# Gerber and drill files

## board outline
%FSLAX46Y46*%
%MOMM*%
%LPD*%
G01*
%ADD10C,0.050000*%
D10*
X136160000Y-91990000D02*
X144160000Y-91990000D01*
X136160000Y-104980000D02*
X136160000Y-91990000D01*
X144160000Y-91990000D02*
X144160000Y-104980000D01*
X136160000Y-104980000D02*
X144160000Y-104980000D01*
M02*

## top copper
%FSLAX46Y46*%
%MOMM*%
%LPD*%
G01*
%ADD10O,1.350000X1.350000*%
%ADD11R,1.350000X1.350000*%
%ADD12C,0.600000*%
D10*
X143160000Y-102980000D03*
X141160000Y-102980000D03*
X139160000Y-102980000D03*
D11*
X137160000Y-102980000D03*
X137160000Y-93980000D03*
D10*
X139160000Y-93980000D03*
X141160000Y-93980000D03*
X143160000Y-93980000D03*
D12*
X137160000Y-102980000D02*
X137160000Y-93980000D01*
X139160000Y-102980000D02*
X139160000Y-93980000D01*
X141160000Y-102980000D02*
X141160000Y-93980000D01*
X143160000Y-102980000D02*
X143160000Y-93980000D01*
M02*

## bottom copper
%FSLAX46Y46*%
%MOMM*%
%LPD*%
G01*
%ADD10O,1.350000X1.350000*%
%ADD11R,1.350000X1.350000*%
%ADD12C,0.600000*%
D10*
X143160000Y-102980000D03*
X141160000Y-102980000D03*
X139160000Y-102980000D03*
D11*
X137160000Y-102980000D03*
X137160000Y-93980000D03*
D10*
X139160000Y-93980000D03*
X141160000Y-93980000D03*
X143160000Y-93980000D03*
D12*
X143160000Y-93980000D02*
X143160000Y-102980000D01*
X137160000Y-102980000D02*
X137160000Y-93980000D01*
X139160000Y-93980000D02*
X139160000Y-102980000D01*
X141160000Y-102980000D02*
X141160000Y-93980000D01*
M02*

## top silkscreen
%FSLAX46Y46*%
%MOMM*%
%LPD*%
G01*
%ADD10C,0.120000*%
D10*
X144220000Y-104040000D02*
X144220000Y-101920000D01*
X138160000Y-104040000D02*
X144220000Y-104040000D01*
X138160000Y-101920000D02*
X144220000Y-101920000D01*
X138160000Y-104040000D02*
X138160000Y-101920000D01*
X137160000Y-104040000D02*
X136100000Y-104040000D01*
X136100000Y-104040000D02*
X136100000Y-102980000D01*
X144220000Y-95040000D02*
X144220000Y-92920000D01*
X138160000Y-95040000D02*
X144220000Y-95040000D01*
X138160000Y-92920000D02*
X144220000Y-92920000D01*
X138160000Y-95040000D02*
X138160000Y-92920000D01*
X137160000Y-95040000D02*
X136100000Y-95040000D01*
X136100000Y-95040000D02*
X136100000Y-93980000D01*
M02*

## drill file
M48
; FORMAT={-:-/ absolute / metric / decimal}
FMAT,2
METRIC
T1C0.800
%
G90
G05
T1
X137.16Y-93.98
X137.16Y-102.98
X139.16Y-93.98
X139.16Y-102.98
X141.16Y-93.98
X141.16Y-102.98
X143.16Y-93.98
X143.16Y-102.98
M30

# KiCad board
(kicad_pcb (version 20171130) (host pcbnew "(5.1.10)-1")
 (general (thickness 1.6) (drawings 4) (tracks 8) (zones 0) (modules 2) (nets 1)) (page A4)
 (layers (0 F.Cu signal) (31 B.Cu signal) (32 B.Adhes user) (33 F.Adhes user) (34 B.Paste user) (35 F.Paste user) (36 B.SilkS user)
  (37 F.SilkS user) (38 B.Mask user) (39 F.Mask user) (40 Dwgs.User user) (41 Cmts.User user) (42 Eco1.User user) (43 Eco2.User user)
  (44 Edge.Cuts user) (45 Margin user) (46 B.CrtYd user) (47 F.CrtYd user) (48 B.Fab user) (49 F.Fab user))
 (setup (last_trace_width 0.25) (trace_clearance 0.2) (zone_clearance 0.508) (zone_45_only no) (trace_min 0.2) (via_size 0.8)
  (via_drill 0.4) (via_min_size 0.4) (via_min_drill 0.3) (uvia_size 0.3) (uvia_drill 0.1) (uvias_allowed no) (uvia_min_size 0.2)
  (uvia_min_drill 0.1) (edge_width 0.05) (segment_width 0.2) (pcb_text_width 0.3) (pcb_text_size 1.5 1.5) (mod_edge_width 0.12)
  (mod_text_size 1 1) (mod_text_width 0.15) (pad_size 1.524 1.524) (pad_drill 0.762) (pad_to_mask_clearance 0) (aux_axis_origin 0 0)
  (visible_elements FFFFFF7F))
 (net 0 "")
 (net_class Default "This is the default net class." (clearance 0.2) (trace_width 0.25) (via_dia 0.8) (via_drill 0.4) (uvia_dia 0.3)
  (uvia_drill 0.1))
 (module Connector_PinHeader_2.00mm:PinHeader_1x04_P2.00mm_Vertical (layer F.Cu) (at 137.16 102.98 90)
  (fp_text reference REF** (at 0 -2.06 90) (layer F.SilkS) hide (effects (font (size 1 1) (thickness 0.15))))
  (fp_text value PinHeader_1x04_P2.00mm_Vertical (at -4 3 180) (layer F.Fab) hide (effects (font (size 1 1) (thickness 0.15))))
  (fp_line (start -1.06 7.06) (end 1.06 7.06) (layer F.SilkS) (width 0.12))
  (fp_line (start -1.06 1) (end -1.06 7.06) (layer F.SilkS) (width 0.12))
  (fp_line (start 1.06 1) (end 1.06 7.06) (layer F.SilkS) (width 0.12))
  (fp_line (start -1.06 1) (end 1.06 1) (layer F.SilkS) (width 0.12))
  (fp_line (start -1.06 0) (end -1.06 -1.06) (layer F.SilkS) (width 0.12))
  (fp_line (start -1.06 -1.06) (end 0 -1.06) (layer F.SilkS) (width 0.12))
  (pad 4 thru_hole oval (at 0 6 90) (size 1.35 1.35) (drill 0.8) (layers *.Cu *.Mask))
  (pad 3 thru_hole oval (at 0 4 90) (size 1.35 1.35) (drill 0.8) (layers *.Cu *.Mask))
  (pad 2 thru_hole oval (at 0 2 90) (size 1.35 1.35) (drill 0.8) (layers *.Cu *.Mask))
  (pad 1 thru_hole rect (at 0 0 90) (size 1.35 1.35) (drill 0.8) (layers *.Cu *.Mask)))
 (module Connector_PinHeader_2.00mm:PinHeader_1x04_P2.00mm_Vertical (layer F.Cu) (at 137.16 93.98 90)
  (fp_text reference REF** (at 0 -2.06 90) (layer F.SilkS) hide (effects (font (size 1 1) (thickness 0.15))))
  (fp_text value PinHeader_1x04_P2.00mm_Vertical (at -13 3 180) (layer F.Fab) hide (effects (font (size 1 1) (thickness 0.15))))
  (fp_line (start -1.06 7.06) (end 1.06 7.06) (layer F.SilkS) (width 0.12))
  (fp_line (start -1.06 1) (end -1.06 7.06) (layer F.SilkS) (width 0.12))
  (fp_line (start 1.06 1) (end 1.06 7.06) (layer F.SilkS) (width 0.12))
  (fp_line (start -1.06 1) (end 1.06 1) (layer F.SilkS) (width 0.12))
  (fp_line (start -1.06 0) (end -1.06 -1.06) (layer F.SilkS) (width 0.12))
  (fp_line (start -1.06 -1.06) (end 0 -1.06) (layer F.SilkS) (width 0.12))
  (pad 1 thru_hole rect (at 0 0 90) (size 1.35 1.35) (drill 0.8) (layers *.Cu *.Mask))
  (pad 2 thru_hole oval (at 0 2 90) (size 1.35 1.35) (drill 0.8) (layers *.Cu *.Mask))
  (pad 3 thru_hole oval (at 0 4 90) (size 1.35 1.35) (drill 0.8) (layers *.Cu *.Mask))
  (pad 4 thru_hole oval (at 0 6 90) (size 1.35 1.35) (drill 0.8) (layers *.Cu *.Mask)))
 (gr_line (start 136.16 91.99) (end 144.16 91.99) (layer Edge.Cuts) (width 0.05))
 (gr_line (start 136.16 104.98) (end 136.16 91.99) (layer Edge.Cuts) (width 0.05))
 (gr_line (start 144.16 91.99) (end 144.16 104.98) (layer Edge.Cuts) (width 0.05))
 (gr_line (start 136.16 104.98) (end 144.16 104.98) (layer Edge.Cuts) (width 0.05))
 (segment (start 143.16 93.98) (end 143.16 102.98) (width 0.6) (layer B.Cu) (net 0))
 (segment (start 137.16 102.98) (end 137.16 93.98) (width 0.6) (layer B.Cu) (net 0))
 (segment (start 139.16 93.98) (end 139.16 102.98) (width 0.6) (layer B.Cu) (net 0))
 (segment (start 141.16 102.98) (end 141.16 93.98) (width 0.6) (layer B.Cu) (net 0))
 (segment (start 137.16 102.98) (end 137.16 93.98) (width 0.6) (layer F.Cu) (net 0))
 (segment (start 139.16 102.98) (end 139.16 93.98) (width 0.6) (layer F.Cu) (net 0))
 (segment (start 141.16 102.98) (end 141.16 93.98) (width 0.6) (layer F.Cu) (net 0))
 (segment (start 143.16 102.98) (end 143.16 93.98) (width 0.6) (layer F.Cu) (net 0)))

